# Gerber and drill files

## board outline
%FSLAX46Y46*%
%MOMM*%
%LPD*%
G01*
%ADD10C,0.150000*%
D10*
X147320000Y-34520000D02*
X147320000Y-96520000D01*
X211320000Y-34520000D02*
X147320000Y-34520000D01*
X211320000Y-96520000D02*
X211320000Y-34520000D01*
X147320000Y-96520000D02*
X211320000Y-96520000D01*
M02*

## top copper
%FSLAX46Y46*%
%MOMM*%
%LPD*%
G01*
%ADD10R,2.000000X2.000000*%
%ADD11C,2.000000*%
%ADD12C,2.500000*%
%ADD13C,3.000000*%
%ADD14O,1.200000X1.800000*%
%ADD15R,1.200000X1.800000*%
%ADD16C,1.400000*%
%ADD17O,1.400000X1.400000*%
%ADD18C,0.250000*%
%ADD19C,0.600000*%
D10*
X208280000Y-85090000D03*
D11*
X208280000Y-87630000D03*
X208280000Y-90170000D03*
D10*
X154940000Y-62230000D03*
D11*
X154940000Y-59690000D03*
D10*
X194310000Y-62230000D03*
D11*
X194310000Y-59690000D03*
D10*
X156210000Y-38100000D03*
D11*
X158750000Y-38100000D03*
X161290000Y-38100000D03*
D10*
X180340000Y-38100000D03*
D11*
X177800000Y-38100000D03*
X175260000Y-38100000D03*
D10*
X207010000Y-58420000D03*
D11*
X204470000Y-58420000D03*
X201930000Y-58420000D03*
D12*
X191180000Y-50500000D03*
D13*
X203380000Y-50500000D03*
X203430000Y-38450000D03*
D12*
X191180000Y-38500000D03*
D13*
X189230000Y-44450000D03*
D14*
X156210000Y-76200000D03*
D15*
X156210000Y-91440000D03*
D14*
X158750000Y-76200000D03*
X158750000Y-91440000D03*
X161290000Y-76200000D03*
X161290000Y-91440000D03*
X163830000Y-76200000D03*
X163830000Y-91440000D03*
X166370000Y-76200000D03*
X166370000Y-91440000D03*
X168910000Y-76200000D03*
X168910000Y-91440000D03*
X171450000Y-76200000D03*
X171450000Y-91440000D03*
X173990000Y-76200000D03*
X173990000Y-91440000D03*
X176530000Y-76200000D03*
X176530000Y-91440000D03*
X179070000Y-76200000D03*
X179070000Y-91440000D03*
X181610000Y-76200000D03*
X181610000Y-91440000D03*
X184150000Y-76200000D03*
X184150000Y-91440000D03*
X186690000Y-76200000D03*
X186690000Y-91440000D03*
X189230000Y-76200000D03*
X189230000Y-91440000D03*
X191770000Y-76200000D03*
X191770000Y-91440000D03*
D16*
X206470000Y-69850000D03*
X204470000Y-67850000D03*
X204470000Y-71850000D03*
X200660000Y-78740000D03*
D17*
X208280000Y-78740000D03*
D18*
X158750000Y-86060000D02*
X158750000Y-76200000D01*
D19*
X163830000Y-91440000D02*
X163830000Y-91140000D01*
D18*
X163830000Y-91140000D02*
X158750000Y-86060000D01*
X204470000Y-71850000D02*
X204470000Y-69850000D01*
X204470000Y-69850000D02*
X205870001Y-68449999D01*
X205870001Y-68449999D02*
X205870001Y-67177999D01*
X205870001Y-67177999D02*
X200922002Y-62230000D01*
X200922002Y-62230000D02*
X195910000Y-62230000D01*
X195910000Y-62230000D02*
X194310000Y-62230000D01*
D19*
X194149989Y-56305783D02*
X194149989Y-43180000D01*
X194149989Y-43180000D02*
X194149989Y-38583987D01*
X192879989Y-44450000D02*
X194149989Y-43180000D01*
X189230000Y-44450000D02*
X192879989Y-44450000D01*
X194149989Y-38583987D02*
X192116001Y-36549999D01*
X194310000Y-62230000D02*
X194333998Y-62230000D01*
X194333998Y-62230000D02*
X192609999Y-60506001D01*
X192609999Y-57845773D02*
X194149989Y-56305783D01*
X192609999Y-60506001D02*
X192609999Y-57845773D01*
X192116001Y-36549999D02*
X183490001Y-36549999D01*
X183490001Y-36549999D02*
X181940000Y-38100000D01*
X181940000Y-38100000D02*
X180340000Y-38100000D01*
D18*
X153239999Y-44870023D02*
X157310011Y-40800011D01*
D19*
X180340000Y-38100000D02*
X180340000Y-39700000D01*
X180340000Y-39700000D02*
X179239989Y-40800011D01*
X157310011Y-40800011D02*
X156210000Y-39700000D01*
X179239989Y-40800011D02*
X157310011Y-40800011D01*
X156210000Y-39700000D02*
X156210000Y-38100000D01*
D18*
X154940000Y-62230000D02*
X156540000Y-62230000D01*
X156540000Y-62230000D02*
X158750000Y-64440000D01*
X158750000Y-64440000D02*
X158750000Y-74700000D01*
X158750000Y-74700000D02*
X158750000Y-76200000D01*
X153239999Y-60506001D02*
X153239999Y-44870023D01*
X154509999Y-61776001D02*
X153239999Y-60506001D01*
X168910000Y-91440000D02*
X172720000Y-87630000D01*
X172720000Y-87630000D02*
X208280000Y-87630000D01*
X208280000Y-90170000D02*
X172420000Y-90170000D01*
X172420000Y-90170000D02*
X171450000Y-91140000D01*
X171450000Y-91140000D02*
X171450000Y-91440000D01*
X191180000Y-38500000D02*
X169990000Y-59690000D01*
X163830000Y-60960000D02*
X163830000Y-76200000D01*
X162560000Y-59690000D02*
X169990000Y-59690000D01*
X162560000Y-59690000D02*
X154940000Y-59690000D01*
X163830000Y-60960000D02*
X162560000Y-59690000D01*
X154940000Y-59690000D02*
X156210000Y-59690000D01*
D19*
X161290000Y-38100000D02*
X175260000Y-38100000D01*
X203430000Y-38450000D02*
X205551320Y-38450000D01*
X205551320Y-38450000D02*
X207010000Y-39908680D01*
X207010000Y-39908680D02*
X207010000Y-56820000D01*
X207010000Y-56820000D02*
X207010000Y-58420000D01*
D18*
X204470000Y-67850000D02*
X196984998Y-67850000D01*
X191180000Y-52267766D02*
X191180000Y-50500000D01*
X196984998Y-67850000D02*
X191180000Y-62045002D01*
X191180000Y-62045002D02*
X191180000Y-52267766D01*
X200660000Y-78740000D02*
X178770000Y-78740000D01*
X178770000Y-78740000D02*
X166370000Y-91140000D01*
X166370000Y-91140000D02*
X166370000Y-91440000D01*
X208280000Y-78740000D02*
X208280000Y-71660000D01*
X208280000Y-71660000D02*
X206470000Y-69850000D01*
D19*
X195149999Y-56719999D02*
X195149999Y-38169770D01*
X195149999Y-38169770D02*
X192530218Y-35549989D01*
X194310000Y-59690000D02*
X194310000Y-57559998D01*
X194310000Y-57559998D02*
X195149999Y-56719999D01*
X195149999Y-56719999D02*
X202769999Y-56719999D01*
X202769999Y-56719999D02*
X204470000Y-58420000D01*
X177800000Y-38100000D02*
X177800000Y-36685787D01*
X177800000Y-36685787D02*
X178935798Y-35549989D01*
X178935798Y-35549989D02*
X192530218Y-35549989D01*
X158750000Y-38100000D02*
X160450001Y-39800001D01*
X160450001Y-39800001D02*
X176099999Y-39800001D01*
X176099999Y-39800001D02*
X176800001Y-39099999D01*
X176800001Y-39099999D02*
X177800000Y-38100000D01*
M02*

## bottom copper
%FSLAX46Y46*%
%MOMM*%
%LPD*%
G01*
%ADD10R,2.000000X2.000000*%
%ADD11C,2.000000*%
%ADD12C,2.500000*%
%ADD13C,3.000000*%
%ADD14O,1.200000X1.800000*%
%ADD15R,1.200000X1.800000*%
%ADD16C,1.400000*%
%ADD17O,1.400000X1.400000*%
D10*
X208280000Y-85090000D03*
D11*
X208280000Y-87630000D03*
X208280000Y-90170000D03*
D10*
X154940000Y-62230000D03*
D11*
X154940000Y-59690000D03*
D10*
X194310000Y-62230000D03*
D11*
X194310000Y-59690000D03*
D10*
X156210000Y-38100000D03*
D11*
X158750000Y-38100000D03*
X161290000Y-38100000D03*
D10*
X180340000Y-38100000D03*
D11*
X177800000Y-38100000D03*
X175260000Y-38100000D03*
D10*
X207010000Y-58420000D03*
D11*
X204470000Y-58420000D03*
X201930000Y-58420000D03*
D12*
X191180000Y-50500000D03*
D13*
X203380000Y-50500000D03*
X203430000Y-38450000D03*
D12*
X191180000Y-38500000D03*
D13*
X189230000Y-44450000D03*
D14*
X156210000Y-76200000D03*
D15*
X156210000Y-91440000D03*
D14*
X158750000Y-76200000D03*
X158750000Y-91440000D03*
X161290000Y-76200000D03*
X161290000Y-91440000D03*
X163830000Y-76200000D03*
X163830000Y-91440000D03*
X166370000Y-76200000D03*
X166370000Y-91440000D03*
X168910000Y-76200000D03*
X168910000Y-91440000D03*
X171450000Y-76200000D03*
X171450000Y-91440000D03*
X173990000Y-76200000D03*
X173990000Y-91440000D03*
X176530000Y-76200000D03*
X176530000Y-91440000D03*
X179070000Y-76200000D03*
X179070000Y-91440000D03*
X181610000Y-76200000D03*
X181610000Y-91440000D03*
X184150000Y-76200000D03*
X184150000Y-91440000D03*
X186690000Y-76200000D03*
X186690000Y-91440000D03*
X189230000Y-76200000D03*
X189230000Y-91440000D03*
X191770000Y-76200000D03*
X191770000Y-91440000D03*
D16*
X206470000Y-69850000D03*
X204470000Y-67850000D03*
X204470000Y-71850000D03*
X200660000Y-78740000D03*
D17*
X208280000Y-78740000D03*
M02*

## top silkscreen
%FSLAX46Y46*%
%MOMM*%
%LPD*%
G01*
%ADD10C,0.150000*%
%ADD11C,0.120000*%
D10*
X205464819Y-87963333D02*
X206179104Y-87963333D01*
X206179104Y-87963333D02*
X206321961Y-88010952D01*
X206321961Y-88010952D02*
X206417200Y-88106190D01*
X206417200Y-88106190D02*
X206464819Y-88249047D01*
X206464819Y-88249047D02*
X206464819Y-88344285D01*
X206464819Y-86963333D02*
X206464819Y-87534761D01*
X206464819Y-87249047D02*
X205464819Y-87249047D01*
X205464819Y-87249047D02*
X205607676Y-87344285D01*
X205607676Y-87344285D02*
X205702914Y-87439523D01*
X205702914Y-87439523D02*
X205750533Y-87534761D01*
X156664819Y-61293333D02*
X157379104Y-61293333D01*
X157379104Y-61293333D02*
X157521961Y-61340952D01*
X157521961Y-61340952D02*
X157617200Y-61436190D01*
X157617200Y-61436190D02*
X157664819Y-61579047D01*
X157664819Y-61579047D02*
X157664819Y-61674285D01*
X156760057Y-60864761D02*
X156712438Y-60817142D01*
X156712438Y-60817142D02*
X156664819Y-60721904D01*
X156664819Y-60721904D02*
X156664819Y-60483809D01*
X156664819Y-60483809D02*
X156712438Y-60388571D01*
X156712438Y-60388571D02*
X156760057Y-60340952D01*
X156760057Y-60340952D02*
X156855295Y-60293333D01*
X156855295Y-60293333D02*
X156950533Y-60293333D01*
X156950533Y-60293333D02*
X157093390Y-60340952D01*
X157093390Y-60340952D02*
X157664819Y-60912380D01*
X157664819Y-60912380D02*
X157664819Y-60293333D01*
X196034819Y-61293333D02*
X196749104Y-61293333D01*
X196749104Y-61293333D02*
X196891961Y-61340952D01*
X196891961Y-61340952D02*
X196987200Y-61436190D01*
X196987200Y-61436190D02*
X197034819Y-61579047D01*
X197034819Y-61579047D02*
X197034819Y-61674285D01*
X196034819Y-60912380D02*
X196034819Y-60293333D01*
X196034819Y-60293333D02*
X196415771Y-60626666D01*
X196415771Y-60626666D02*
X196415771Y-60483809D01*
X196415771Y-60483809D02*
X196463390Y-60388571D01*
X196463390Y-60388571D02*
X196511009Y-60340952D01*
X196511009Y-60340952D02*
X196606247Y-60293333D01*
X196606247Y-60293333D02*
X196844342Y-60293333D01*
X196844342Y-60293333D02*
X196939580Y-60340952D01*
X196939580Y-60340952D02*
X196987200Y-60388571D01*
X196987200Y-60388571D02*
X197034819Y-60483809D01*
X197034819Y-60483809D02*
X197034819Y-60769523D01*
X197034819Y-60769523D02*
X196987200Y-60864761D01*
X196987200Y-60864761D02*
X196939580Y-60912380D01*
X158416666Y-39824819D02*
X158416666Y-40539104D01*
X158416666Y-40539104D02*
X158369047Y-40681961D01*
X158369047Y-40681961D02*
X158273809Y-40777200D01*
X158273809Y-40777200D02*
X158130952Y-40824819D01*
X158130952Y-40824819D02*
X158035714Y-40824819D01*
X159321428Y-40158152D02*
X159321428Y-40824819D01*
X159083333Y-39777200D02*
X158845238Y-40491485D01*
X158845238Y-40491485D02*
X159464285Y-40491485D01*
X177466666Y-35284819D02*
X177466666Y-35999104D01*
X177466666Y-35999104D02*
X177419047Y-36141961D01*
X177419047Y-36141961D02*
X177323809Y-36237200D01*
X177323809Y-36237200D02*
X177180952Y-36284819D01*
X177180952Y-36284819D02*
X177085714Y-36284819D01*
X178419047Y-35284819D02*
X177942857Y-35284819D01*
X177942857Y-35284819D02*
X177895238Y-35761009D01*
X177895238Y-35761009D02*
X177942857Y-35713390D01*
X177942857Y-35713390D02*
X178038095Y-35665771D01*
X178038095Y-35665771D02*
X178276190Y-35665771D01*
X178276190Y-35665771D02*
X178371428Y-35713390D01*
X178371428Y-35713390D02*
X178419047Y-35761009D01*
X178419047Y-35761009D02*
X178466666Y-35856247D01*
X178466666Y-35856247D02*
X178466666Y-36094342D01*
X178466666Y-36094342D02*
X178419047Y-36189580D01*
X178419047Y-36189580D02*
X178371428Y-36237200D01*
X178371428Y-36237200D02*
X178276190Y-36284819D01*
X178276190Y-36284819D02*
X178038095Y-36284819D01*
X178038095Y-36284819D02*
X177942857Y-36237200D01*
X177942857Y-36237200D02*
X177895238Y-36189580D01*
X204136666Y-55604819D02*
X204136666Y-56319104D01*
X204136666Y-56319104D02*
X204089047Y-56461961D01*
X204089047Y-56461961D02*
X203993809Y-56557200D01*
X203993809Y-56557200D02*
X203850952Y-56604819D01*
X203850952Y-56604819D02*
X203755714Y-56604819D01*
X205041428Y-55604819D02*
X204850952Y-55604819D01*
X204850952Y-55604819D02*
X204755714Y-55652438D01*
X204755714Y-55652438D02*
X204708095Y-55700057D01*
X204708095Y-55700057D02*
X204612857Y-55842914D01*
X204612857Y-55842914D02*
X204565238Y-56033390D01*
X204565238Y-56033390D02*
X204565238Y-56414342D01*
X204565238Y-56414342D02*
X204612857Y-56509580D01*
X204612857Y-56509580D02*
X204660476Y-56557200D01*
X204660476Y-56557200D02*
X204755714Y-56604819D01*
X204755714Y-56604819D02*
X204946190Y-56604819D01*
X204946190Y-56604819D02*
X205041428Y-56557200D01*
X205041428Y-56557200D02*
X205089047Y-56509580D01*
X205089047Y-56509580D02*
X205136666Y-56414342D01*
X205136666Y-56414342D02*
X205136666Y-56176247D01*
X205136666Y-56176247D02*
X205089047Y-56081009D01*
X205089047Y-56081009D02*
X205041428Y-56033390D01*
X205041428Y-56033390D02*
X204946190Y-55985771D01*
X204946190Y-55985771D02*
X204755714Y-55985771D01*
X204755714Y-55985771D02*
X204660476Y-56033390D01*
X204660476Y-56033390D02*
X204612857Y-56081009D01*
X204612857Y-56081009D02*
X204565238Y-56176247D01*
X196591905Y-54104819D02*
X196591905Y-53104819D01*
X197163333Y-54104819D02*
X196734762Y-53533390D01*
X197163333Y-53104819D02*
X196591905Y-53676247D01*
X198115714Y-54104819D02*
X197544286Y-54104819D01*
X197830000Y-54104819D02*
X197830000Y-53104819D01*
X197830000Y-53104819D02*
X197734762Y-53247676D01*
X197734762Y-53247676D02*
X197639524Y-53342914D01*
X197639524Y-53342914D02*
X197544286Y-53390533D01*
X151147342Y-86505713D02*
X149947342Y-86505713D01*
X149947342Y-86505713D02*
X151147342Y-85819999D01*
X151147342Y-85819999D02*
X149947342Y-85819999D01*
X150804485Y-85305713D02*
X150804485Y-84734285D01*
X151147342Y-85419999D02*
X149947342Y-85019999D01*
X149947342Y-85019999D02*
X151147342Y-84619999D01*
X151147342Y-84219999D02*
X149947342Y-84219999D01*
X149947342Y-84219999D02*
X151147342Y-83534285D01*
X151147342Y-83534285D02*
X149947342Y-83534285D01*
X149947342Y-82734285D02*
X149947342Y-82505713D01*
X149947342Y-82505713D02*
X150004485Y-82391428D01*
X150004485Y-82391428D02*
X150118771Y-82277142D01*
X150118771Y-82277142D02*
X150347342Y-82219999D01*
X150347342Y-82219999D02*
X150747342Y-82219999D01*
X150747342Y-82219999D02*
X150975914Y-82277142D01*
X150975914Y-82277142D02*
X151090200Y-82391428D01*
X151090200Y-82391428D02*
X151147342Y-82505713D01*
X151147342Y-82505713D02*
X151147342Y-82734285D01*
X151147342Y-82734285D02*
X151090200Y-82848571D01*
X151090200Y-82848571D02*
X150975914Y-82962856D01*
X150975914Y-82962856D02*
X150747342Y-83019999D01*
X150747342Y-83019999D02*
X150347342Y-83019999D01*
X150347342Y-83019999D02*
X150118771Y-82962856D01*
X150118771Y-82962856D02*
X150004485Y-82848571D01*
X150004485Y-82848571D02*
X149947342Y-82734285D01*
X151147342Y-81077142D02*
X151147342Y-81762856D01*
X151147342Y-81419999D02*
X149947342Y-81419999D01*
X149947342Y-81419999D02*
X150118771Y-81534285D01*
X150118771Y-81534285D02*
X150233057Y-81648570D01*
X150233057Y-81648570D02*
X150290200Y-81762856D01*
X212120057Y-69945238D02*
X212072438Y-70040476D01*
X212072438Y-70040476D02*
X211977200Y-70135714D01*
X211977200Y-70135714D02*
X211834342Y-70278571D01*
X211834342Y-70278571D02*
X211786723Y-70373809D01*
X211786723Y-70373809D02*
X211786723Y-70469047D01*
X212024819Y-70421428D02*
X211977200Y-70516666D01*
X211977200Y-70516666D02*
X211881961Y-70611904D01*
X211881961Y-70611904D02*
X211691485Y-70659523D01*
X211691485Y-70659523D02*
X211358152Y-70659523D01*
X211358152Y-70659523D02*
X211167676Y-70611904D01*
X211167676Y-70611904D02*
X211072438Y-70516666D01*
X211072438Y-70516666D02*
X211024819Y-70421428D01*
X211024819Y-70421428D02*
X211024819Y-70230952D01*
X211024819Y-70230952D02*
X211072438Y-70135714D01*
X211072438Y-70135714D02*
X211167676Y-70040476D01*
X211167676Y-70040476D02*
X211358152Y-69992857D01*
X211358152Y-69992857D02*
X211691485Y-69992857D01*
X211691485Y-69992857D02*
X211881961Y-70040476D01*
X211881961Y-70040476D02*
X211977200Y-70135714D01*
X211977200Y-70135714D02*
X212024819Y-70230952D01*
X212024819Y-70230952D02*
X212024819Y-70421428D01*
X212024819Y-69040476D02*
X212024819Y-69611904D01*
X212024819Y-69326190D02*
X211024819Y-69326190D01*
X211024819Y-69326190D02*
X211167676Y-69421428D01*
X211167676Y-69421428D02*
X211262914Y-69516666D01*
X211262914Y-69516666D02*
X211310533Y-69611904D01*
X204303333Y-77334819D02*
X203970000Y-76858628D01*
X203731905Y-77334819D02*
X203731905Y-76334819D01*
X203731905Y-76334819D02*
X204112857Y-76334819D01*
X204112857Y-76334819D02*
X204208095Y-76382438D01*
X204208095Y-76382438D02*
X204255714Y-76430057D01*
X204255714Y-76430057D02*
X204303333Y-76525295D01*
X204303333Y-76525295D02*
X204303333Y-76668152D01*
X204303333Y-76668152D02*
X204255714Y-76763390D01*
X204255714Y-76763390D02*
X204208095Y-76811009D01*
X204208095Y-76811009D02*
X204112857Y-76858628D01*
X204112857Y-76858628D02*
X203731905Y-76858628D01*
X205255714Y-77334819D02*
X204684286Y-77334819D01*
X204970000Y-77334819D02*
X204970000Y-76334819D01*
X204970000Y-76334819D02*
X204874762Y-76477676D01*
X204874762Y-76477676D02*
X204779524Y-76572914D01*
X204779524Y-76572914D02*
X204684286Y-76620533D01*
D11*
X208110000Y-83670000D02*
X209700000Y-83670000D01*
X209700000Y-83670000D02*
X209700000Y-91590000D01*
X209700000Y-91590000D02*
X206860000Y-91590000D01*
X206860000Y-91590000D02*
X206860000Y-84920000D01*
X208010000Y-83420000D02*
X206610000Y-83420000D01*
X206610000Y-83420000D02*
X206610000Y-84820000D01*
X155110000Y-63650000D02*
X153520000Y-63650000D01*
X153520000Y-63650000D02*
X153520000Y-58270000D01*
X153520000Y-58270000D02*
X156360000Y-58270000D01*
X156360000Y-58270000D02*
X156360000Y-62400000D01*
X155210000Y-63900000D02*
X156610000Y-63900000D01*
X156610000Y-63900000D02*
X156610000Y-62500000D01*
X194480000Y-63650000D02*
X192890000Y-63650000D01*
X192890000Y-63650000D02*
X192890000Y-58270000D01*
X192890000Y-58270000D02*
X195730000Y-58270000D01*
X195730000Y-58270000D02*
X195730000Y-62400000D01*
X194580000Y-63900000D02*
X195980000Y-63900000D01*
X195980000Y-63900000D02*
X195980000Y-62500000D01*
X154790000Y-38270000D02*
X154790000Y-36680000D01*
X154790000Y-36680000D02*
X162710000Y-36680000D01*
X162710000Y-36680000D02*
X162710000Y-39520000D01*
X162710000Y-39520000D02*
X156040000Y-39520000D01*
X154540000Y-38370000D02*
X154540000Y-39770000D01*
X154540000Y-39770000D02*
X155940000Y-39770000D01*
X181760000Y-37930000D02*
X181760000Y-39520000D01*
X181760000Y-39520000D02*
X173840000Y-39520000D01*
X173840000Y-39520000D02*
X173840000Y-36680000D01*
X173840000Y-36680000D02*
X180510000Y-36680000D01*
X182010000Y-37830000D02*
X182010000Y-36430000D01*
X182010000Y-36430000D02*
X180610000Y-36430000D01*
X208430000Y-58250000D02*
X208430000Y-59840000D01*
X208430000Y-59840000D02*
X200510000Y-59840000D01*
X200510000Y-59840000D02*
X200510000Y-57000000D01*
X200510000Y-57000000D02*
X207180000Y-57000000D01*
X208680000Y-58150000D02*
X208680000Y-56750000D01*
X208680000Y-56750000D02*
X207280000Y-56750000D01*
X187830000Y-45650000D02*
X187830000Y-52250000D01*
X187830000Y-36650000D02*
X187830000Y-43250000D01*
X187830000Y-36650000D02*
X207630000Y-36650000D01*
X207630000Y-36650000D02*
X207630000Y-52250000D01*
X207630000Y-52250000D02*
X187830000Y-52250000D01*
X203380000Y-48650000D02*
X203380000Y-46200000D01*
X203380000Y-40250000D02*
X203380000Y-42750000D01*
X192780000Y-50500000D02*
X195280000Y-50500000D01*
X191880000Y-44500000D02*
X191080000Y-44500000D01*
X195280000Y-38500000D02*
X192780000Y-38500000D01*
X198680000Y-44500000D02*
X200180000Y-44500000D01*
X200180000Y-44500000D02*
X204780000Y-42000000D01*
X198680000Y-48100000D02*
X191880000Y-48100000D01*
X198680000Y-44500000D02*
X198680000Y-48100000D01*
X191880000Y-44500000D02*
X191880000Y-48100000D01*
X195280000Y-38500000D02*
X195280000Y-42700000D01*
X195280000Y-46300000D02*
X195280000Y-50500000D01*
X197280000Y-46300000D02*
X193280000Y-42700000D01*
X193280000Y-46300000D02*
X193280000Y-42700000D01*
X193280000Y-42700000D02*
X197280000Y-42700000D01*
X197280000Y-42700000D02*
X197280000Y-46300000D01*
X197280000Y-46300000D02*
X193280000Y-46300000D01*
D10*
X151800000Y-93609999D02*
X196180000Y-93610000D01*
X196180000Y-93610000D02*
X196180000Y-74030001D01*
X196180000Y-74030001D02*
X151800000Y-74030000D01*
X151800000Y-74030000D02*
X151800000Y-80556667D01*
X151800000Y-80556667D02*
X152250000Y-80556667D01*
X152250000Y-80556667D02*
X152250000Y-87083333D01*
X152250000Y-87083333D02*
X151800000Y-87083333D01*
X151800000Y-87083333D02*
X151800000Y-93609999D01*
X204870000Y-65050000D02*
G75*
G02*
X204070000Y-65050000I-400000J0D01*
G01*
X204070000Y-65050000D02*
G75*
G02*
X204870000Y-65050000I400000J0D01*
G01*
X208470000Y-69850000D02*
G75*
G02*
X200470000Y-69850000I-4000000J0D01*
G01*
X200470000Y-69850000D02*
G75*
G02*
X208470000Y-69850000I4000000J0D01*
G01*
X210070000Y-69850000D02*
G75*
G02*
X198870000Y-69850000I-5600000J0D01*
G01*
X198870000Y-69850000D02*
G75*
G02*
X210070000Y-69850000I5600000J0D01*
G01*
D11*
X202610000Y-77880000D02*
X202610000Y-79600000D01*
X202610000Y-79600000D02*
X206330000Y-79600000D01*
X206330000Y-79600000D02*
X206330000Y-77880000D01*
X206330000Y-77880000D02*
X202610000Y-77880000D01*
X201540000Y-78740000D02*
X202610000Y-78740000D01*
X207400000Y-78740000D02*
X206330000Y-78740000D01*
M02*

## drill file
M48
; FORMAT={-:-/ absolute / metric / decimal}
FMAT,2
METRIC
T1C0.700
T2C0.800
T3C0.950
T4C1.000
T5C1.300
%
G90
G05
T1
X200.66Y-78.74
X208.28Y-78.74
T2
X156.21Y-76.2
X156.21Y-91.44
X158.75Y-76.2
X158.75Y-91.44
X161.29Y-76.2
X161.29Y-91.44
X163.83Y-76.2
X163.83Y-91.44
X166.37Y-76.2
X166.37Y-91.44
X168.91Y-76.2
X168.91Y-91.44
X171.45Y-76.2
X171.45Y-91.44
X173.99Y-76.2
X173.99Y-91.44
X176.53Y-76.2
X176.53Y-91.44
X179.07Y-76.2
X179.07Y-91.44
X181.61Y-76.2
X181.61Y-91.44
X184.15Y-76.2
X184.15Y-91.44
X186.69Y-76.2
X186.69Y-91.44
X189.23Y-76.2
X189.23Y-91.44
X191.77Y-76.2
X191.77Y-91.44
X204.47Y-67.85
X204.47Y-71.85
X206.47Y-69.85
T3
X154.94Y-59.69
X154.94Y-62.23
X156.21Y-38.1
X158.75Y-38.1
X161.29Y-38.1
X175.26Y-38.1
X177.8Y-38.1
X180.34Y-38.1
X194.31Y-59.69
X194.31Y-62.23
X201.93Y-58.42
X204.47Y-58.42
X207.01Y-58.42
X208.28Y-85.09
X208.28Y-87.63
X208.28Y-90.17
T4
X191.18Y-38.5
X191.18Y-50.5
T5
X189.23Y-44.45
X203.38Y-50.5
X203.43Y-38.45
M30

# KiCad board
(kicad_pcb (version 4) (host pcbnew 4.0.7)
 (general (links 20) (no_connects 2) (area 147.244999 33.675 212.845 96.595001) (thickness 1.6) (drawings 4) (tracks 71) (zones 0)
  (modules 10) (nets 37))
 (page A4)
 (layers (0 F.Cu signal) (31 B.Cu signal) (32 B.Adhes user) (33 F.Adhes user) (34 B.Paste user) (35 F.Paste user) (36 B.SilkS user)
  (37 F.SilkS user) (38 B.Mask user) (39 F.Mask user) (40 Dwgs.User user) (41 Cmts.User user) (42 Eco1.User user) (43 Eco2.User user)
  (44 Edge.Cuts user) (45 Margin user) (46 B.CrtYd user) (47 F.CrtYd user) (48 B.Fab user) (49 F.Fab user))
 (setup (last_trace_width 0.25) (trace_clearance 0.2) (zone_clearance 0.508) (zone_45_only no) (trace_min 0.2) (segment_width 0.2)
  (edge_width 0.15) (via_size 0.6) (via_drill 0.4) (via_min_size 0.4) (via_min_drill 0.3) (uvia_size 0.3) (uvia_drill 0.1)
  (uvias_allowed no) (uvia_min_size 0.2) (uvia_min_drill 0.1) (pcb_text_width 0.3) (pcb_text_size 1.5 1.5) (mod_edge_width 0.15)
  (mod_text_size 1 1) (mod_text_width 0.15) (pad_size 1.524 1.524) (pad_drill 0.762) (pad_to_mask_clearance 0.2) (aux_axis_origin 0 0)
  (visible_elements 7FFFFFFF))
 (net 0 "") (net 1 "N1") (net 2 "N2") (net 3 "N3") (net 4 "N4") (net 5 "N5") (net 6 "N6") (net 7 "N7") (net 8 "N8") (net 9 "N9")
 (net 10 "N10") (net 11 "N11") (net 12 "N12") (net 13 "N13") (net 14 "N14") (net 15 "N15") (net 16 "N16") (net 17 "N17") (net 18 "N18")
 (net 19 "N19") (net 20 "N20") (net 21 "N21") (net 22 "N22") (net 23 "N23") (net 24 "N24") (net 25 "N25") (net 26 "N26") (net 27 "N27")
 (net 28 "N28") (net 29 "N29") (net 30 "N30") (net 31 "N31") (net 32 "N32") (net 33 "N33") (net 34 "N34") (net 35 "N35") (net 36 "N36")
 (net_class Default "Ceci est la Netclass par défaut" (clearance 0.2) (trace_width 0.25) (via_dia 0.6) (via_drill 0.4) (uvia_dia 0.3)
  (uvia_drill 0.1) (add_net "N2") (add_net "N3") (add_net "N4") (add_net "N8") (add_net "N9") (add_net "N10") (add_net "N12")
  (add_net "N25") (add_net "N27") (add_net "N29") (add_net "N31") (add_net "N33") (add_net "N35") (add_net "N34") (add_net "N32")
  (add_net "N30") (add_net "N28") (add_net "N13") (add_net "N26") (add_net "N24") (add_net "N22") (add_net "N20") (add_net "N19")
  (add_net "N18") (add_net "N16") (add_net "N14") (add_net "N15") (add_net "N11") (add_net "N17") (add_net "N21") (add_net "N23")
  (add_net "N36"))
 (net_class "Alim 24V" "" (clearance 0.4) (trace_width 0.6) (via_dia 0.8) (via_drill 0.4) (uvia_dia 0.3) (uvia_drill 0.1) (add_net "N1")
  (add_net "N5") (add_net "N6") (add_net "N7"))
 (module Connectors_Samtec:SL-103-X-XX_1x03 (layer F.Cu) (at 208.28 85.09)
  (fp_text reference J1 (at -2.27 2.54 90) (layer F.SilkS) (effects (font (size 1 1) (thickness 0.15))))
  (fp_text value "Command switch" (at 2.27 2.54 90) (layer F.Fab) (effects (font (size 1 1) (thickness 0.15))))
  (fp_line (start -0.17 -1.42) (end 1.42 -1.42) (layer F.SilkS) (width 0.12))
  (fp_line (start 1.42 -1.42) (end 1.42 6.5) (layer F.SilkS) (width 0.12))
  (fp_line (start 1.42 6.5) (end -1.42 6.5) (layer F.SilkS) (width 0.12))
  (fp_line (start -1.42 6.5) (end -1.42 -0.17) (layer F.SilkS) (width 0.12))
  (fp_line (start -0.27 -1.67) (end -1.67 -1.67) (layer F.SilkS) (width 0.12))
  (fp_line (start -1.67 -1.67) (end -1.67 -0.27) (layer F.SilkS) (width 0.12))
  (pad 1 thru_hole rect (at 0 0) (size 2 2) (drill 0.95) (layers *.Cu *.Mask) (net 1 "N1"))
  (pad 2 thru_hole circle (at 0 2.54) (size 2 2) (drill 0.95) (layers *.Cu *.Mask) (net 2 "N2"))
  (pad 3 thru_hole circle (at 0 5.08) (size 2 2) (drill 0.95) (layers *.Cu *.Mask) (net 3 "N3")))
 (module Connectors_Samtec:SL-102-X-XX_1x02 (layer F.Cu) (at 154.94 62.23 180)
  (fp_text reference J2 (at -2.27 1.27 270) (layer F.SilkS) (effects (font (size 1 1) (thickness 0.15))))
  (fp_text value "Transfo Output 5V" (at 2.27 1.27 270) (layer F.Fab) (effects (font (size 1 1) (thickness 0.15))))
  (fp_line (start -0.17 -1.42) (end 1.42 -1.42) (layer F.SilkS) (width 0.12))
  (fp_line (start 1.42 -1.42) (end 1.42 3.96) (layer F.SilkS) (width 0.12))
  (fp_line (start 1.42 3.96) (end -1.42 3.96) (layer F.SilkS) (width 0.12))
  (fp_line (start -1.42 3.96) (end -1.42 -0.17) (layer F.SilkS) (width 0.12))
  (fp_line (start -0.27 -1.67) (end -1.67 -1.67) (layer F.SilkS) (width 0.12))
  (fp_line (start -1.67 -1.67) (end -1.67 -0.27) (layer F.SilkS) (width 0.12))
  (pad 1 thru_hole rect (at 0 0 180) (size 2 2) (drill 0.95) (layers *.Cu *.Mask) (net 1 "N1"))
  (pad 2 thru_hole circle (at 0 2.54 180) (size 2 2) (drill 0.95) (layers *.Cu *.Mask) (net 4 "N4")))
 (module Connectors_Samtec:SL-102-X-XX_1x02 (layer F.Cu) (at 194.31 62.23 180)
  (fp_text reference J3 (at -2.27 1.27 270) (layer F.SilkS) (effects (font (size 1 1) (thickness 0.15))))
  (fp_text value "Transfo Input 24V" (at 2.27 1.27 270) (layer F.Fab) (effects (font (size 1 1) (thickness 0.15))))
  (fp_line (start -0.17 -1.42) (end 1.42 -1.42) (layer F.SilkS) (width 0.12))
  (fp_line (start 1.42 -1.42) (end 1.42 3.96) (layer F.SilkS) (width 0.12))
  (fp_line (start 1.42 3.96) (end -1.42 3.96) (layer F.SilkS) (width 0.12))
  (fp_line (start -1.42 3.96) (end -1.42 -0.17) (layer F.SilkS) (width 0.12))
  (fp_line (start -0.27 -1.67) (end -1.67 -1.67) (layer F.SilkS) (width 0.12))
  (fp_line (start -1.67 -1.67) (end -1.67 -0.27) (layer F.SilkS) (width 0.12))
  (pad 1 thru_hole rect (at 0 0 180) (size 2 2) (drill 0.95) (layers *.Cu *.Mask) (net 1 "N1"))
  (pad 2 thru_hole circle (at 0 2.54 180) (size 2 2) (drill 0.95) (layers *.Cu *.Mask) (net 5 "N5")))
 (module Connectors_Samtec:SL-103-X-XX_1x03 (layer F.Cu) (at 156.21 38.1 90)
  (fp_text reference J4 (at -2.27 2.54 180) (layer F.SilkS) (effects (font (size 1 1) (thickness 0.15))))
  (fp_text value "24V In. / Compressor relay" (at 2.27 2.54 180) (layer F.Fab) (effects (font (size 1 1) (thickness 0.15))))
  (fp_line (start -0.17 -1.42) (end 1.42 -1.42) (layer F.SilkS) (width 0.12))
  (fp_line (start 1.42 -1.42) (end 1.42 6.5) (layer F.SilkS) (width 0.12))
  (fp_line (start 1.42 6.5) (end -1.42 6.5) (layer F.SilkS) (width 0.12))
  (fp_line (start -1.42 6.5) (end -1.42 -0.17) (layer F.SilkS) (width 0.12))
  (fp_line (start -0.27 -1.67) (end -1.67 -1.67) (layer F.SilkS) (width 0.12))
  (fp_line (start -1.67 -1.67) (end -1.67 -0.27) (layer F.SilkS) (width 0.12))
  (pad 1 thru_hole rect (at 0 0 90) (size 2 2) (drill 0.95) (layers *.Cu *.Mask) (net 1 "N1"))
  (pad 2 thru_hole circle (at 0 2.54 90) (size 2 2) (drill 0.95) (layers *.Cu *.Mask) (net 5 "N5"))
  (pad 3 thru_hole circle (at 0 5.08 90) (size 2 2) (drill 0.95) (layers *.Cu *.Mask) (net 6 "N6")))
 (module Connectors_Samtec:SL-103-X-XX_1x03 (layer F.Cu) (at 180.34 38.1 270)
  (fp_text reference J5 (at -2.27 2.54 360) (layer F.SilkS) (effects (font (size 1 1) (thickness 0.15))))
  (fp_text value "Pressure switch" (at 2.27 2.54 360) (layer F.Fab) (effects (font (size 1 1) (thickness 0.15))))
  (fp_line (start -0.17 -1.42) (end 1.42 -1.42) (layer F.SilkS) (width 0.12))
  (fp_line (start 1.42 -1.42) (end 1.42 6.5) (layer F.SilkS) (width 0.12))
  (fp_line (start 1.42 6.5) (end -1.42 6.5) (layer F.SilkS) (width 0.12))
  (fp_line (start -1.42 6.5) (end -1.42 -0.17) (layer F.SilkS) (width 0.12))
  (fp_line (start -0.27 -1.67) (end -1.67 -1.67) (layer F.SilkS) (width 0.12))
  (fp_line (start -1.67 -1.67) (end -1.67 -0.27) (layer F.SilkS) (width 0.12))
  (pad 1 thru_hole rect (at 0 0 270) (size 2 2) (drill 0.95) (layers *.Cu *.Mask) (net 1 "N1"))
  (pad 2 thru_hole circle (at 0 2.54 270) (size 2 2) (drill 0.95) (layers *.Cu *.Mask) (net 5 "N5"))
  (pad 3 thru_hole circle (at 0 5.08 270) (size 2 2) (drill 0.95) (layers *.Cu *.Mask) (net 6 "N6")))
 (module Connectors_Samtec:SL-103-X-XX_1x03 (layer F.Cu) (at 207.01 58.42 270)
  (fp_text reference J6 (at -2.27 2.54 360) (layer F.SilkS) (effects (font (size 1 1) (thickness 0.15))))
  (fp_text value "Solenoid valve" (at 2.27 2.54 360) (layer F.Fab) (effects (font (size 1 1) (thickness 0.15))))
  (fp_line (start -0.17 -1.42) (end 1.42 -1.42) (layer F.SilkS) (width 0.12))
  (fp_line (start 1.42 -1.42) (end 1.42 6.5) (layer F.SilkS) (width 0.12))
  (fp_line (start 1.42 6.5) (end -1.42 6.5) (layer F.SilkS) (width 0.12))
  (fp_line (start -1.42 6.5) (end -1.42 -0.17) (layer F.SilkS) (width 0.12))
  (fp_line (start -0.27 -1.67) (end -1.67 -1.67) (layer F.SilkS) (width 0.12))
  (fp_line (start -1.67 -1.67) (end -1.67 -0.27) (layer F.SilkS) (width 0.12))
  (pad 1 thru_hole rect (at 0 0 270) (size 2 2) (drill 0.95) (layers *.Cu *.Mask) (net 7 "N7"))
  (pad 2 thru_hole circle (at 0 2.54 270) (size 2 2) (drill 0.95) (layers *.Cu *.Mask) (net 5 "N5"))
  (pad 3 thru_hole circle (at 0 5.08 270) (size 2 2) (drill 0.95) (layers *.Cu *.Mask) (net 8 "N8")))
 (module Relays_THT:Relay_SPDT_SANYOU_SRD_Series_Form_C (layer F.Cu) (at 189.23 44.45)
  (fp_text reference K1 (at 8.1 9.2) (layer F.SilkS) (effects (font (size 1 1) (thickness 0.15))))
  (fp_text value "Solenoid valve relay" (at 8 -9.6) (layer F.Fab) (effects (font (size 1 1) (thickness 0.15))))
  (fp_line (start -1.4 1.2) (end -1.4 7.8) (layer F.SilkS) (width 0.12))
  (fp_line (start -1.4 -7.8) (end -1.4 -1.2) (layer F.SilkS) (width 0.12))
  (fp_line (start -1.4 -7.8) (end 18.4 -7.8) (layer F.SilkS) (width 0.12))
  (fp_line (start 18.4 -7.8) (end 18.4 7.8) (layer F.SilkS) (width 0.12))
  (fp_line (start 18.4 7.8) (end -1.4 7.8) (layer F.SilkS) (width 0.12))
  (fp_line (start 14.15 4.2) (end 14.15 1.75) (layer F.SilkS) (width 0.12))
  (fp_line (start 14.15 -4.2) (end 14.15 -1.7) (layer F.SilkS) (width 0.12))
  (fp_line (start 3.55 6.05) (end 6.05 6.05) (layer F.SilkS) (width 0.12))
  (fp_line (start 2.65 0.05) (end 1.85 0.05) (layer F.SilkS) (width 0.12))
  (fp_line (start 6.05 -5.95) (end 3.55 -5.95) (layer F.SilkS) (width 0.12))
  (fp_line (start 9.45 0.05) (end 10.95 0.05) (layer F.SilkS) (width 0.12))
  (fp_line (start 10.95 0.05) (end 15.55 -2.45) (layer F.SilkS) (width 0.12))
  (fp_line (start 9.45 3.65) (end 2.65 3.65) (layer F.SilkS) (width 0.12))
  (fp_line (start 9.45 0.05) (end 9.45 3.65) (layer F.SilkS) (width 0.12))
  (fp_line (start 2.65 0.05) (end 2.65 3.65) (layer F.SilkS) (width 0.12))
  (fp_line (start 6.05 -5.95) (end 6.05 -1.75) (layer F.SilkS) (width 0.12))
  (fp_line (start 6.05 1.85) (end 6.05 6.05) (layer F.SilkS) (width 0.12))
  (fp_line (start 8.05 1.85) (end 4.05 -1.75) (layer F.SilkS) (width 0.12))
  (fp_line (start 4.05 1.85) (end 4.05 -1.75) (layer F.SilkS) (width 0.12))
  (fp_line (start 4.05 -1.75) (end 8.05 -1.75) (layer F.SilkS) (width 0.12))
  (fp_line (start 8.05 -1.75) (end 8.05 1.85) (layer F.SilkS) (width 0.12))
  (fp_line (start 8.05 1.85) (end 4.05 1.85) (layer F.SilkS) (width 0.12))
  (pad 2 thru_hole circle (at 1.95 6.05 90) (size 2.5 2.5) (drill 1) (layers *.Cu *.Mask) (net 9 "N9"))
  (pad 3 thru_hole circle (at 14.15 6.05 90) (size 3 3) (drill 1.3) (layers *.Cu *.Mask) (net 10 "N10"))
  (pad 4 thru_hole circle (at 14.2 -6 90) (size 3 3) (drill 1.3) (layers *.Cu *.Mask) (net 7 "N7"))
  (pad 5 thru_hole circle (at 1.95 -5.95 90) (size 2.5 2.5) (drill 1) (layers *.Cu *.Mask) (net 4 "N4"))
  (pad 1 thru_hole circle (at 0 0 90) (size 3 3) (drill 1.3) (layers *.Cu *.Mask) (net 1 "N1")))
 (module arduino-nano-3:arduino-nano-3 (layer F.Cu) (at 173.99 83.82)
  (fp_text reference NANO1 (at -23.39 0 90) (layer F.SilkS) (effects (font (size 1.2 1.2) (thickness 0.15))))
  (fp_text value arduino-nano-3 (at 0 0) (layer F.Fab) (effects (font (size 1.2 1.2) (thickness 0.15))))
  (fp_line (start -22.19 9.789999) (end 22.19 9.79) (layer F.SilkS) (width 0.15))
  (fp_line (start 22.19 9.79) (end 22.19 -9.789999) (layer F.SilkS) (width 0.15))
  (fp_line (start 22.19 -9.789999) (end -22.19 -9.79) (layer F.SilkS) (width 0.15))
  (fp_line (start -22.19 -9.79) (end -22.19 -3.263333) (layer F.SilkS) (width 0.15))
  (fp_line (start -22.19 -3.263333) (end -21.74 -3.263333) (layer F.SilkS) (width 0.15))
  (fp_line (start -21.74 -3.263333) (end -21.74 3.263333) (layer F.SilkS) (width 0.15))
  (fp_line (start -21.74 3.263333) (end -22.19 3.263333) (layer F.SilkS) (width 0.15))
  (fp_line (start -22.19 3.263333) (end -22.19 9.789999) (layer F.SilkS) (width 0.15))
  (pad 30 thru_hole oval (at -17.78 -7.62) (size 1.2 1.8) (drill 0.8) (layers *.Cu *.Mask) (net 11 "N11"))
  (pad 1 thru_hole rect (at -17.78 7.62) (size 1.2 1.8) (drill 0.8) (layers *.Cu *.Mask) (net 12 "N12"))
  (pad 29 thru_hole oval (at -15.24 -7.62) (size 1.2 1.8) (drill 0.8) (layers *.Cu *.Mask) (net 1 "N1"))
  (pad 2 thru_hole oval (at -15.24 7.62) (size 1.2 1.8) (drill 0.8) (layers *.Cu *.Mask) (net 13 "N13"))
  (pad 28 thru_hole oval (at -12.7 -7.62) (size 1.2 1.8) (drill 0.8) (layers *.Cu *.Mask) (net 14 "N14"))
  (pad 3 thru_hole oval (at -12.7 7.62) (size 1.2 1.8) (drill 0.8) (layers *.Cu *.Mask) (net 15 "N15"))
  (pad 27 thru_hole oval (at -10.16 -7.62) (size 1.2 1.8) (drill 0.8) (layers *.Cu *.Mask) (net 4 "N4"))
  (pad 4 thru_hole oval (at -10.16 7.62) (size 1.2 1.8) (drill 0.8) (layers *.Cu *.Mask) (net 1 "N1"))
  (pad 26 thru_hole oval (at -7.62 -7.62) (size 1.2 1.8) (drill 0.8) (layers *.Cu *.Mask) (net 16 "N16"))
  (pad 5 thru_hole oval (at -7.62 7.62) (size 1.2 1.8) (drill 0.8) (layers *.Cu *.Mask) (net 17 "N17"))
  (pad 25 thru_hole oval (at -5.08 -7.62) (size 1.2 1.8) (drill 0.8) (layers *.Cu *.Mask) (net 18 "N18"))
  (pad 6 thru_hole oval (at -5.08 7.62) (size 1.2 1.8) (drill 0.8) (layers *.Cu *.Mask) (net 2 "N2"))
  (pad 24 thru_hole oval (at -2.54 -7.62) (size 1.2 1.8) (drill 0.8) (layers *.Cu *.Mask) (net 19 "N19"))
  (pad 7 thru_hole oval (at -2.54 7.62) (size 1.2 1.8) (drill 0.8) (layers *.Cu *.Mask) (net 3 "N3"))
  (pad 23 thru_hole oval (at 0 -7.62) (size 1.2 1.8) (drill 0.8) (layers *.Cu *.Mask) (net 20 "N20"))
  (pad 8 thru_hole oval (at 0 7.62) (size 1.2 1.8) (drill 0.8) (layers *.Cu *.Mask) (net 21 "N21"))
  (pad 22 thru_hole oval (at 2.54 -7.62) (size 1.2 1.8) (drill 0.8) (layers *.Cu *.Mask) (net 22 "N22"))
  (pad 9 thru_hole oval (at 2.54 7.62) (size 1.2 1.8) (drill 0.8) (layers *.Cu *.Mask) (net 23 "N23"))
  (pad 21 thru_hole oval (at 5.08 -7.62) (size 1.2 1.8) (drill 0.8) (layers *.Cu *.Mask) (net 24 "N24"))
  (pad 10 thru_hole oval (at 5.08 7.62) (size 1.2 1.8) (drill 0.8) (layers *.Cu *.Mask) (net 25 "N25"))
  (pad 20 thru_hole oval (at 7.62 -7.62) (size 1.2 1.8) (drill 0.8) (layers *.Cu *.Mask) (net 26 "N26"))
  (pad 11 thru_hole oval (at 7.62 7.62) (size 1.2 1.8) (drill 0.8) (layers *.Cu *.Mask) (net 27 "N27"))
  (pad 19 thru_hole oval (at 10.16 -7.62) (size 1.2 1.8) (drill 0.8) (layers *.Cu *.Mask) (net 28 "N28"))
  (pad 12 thru_hole oval (at 10.16 7.62) (size 1.2 1.8) (drill 0.8) (layers *.Cu *.Mask) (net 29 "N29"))
  (pad 18 thru_hole oval (at 12.7 -7.62) (size 1.2 1.8) (drill 0.8) (layers *.Cu *.Mask) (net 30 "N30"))
  (pad 13 thru_hole oval (at 12.7 7.62) (size 1.2 1.8) (drill 0.8) (layers *.Cu *.Mask) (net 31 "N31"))
  (pad 17 thru_hole oval (at 15.24 -7.62) (size 1.2 1.8) (drill 0.8) (layers *.Cu *.Mask) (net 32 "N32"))
  (pad 14 thru_hole oval (at 15.24 7.62) (size 1.2 1.8) (drill 0.8) (layers *.Cu *.Mask) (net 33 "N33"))
  (pad 16 thru_hole oval (at 17.78 -7.62) (size 1.2 1.8) (drill 0.8) (layers *.Cu *.Mask) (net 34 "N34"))
  (pad 15 thru_hole oval (at 17.78 7.62) (size 1.2 1.8) (drill 0.8) (layers *.Cu *.Mask) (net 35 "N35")))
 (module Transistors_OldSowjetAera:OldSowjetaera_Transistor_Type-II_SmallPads (layer F.Cu) (at 204.47 69.85 270)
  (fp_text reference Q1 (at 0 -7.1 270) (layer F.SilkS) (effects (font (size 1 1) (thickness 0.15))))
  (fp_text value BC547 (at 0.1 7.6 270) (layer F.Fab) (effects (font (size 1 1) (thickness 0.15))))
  (fp_circle (center -4.8 0) (end -4.8 0.4) (layer F.SilkS) (width 0.15))
  (fp_circle (center 0 0) (end 4 0) (layer F.SilkS) (width 0.15))
  (fp_circle (center 0 0) (end 5.6 0) (layer F.SilkS) (width 0.15))
  (pad 2 thru_hole circle (at 0 -2 270) (size 1.4 1.4) (drill 0.8) (layers *.Cu *.Mask) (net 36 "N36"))
  (pad 1 thru_hole circle (at -2 0 270) (size 1.4 1.4) (drill 0.8) (layers *.Cu *.Mask) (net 9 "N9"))
  (pad 3 thru_hole circle (at 2 0 270) (size 1.4 1.4) (drill 0.8) (layers *.Cu *.Mask) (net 1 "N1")))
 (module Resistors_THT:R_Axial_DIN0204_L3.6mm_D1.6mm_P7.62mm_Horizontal (layer F.Cu) (at 200.66 78.74)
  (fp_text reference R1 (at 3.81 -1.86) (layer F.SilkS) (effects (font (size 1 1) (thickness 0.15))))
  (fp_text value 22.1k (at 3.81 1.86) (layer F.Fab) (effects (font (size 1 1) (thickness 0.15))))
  (fp_line (start 1.95 -0.86) (end 1.95 0.86) (layer F.SilkS) (width 0.12))
  (fp_line (start 1.95 0.86) (end 5.67 0.86) (layer F.SilkS) (width 0.12))
  (fp_line (start 5.67 0.86) (end 5.67 -0.86) (layer F.SilkS) (width 0.12))
  (fp_line (start 5.67 -0.86) (end 1.95 -0.86) (layer F.SilkS) (width 0.12))
  (fp_line (start 0.88 0) (end 1.95 0) (layer F.SilkS) (width 0.12))
  (fp_line (start 6.74 0) (end 5.67 0) (layer F.SilkS) (width 0.12))
  (pad 1 thru_hole circle (at 0 0) (size 1.4 1.4) (drill 0.7) (layers *.Cu *.Mask) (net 17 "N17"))
  (pad 2 thru_hole oval (at 7.62 0) (size 1.4 1.4) (drill 0.7) (layers *.Cu *.Mask) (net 36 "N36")))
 (gr_line (start 147.32 34.52) (end 147.32 96.52) (angle 90) (layer Edge.Cuts) (width 0.15))
 (gr_line (start 211.32 34.52) (end 147.32 34.52) (angle 90) (layer Edge.Cuts) (width 0.15))
 (gr_line (start 211.32 96.52) (end 211.32 34.52) (angle 90) (layer Edge.Cuts) (width 0.15))
 (gr_line (start 147.32 96.52) (end 211.32 96.52) (angle 90) (layer Edge.Cuts) (width 0.15))
 (segment (start 158.75 86.06) (end 158.75 76.2) (width 0.25) (layer F.Cu) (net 1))
 (segment (start 163.83 91.44) (end 163.83 91.14) (width 0.6) (layer F.Cu) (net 1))
 (segment (start 163.83 91.14) (end 158.75 86.06) (width 0.25) (layer F.Cu) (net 1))
 (segment (start 204.47 71.85) (end 204.47 69.85) (width 0.25) (layer F.Cu) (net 1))
 (segment (start 204.47 69.85) (end 205.870001 68.449999) (width 0.25) (layer F.Cu) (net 1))
 (segment (start 205.870001 68.449999) (end 205.870001 67.177999) (width 0.25) (layer F.Cu) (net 1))
 (segment (start 205.870001 67.177999) (end 200.922002 62.23) (width 0.25) (layer F.Cu) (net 1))
 (segment (start 200.922002 62.23) (end 195.91 62.23) (width 0.25) (layer F.Cu) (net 1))
 (segment (start 195.91 62.23) (end 194.31 62.23) (width 0.25) (layer F.Cu) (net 1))
 (segment (start 194.149989 56.305783) (end 194.149989 43.18) (width 0.6) (layer F.Cu) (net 1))
 (segment (start 194.149989 43.18) (end 194.149989 38.583987) (width 0.6) (layer F.Cu) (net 1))
 (segment (start 192.879989 44.45) (end 194.149989 43.18) (width 0.6) (layer F.Cu) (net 1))
 (segment (start 189.23 44.45) (end 192.879989 44.45) (width 0.6) (layer F.Cu) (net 1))
 (segment (start 194.149989 38.583987) (end 192.116001 36.549999) (width 0.6) (layer F.Cu) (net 1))
 (segment (start 194.31 62.23) (end 194.333998 62.23) (width 0.6) (layer F.Cu) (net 1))
 (segment (start 194.333998 62.23) (end 192.609999 60.506001) (width 0.6) (layer F.Cu) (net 1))
 (segment (start 192.609999 57.845773) (end 194.149989 56.305783) (width 0.6) (layer F.Cu) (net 1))
 (segment (start 192.609999 60.506001) (end 192.609999 57.845773) (width 0.6) (layer F.Cu) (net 1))
 (segment (start 192.116001 36.549999) (end 183.490001 36.549999) (width 0.6) (layer F.Cu) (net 1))
 (segment (start 183.490001 36.549999) (end 181.94 38.1) (width 0.6) (layer F.Cu) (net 1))
 (segment (start 181.94 38.1) (end 180.34 38.1) (width 0.6) (layer F.Cu) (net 1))
 (segment (start 153.239999 44.870023) (end 157.310011 40.800011) (width 0.25) (layer F.Cu) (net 1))
 (segment (start 180.34 38.1) (end 180.34 39.7) (width 0.6) (layer F.Cu) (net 1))
 (segment (start 180.34 39.7) (end 179.239989 40.800011) (width 0.6) (layer F.Cu) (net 1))
 (segment (start 157.310011 40.800011) (end 156.21 39.7) (width 0.6) (layer F.Cu) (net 1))
 (segment (start 179.239989 40.800011) (end 157.310011 40.800011) (width 0.6) (layer F.Cu) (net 1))
 (segment (start 156.21 39.7) (end 156.21 38.1) (width 0.6) (layer F.Cu) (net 1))
 (segment (start 154.94 62.23) (end 156.54 62.23) (width 0.25) (layer F.Cu) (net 1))
 (segment (start 156.54 62.23) (end 158.75 64.44) (width 0.25) (layer F.Cu) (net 1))
 (segment (start 158.75 64.44) (end 158.75 74.7) (width 0.25) (layer F.Cu) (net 1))
 (segment (start 158.75 74.7) (end 158.75 76.2) (width 0.25) (layer F.Cu) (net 1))
 (segment (start 153.239999 60.506001) (end 153.239999 44.870023) (width 0.25) (layer F.Cu) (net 1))
 (segment (start 154.509999 61.776001) (end 153.239999 60.506001) (width 0.25) (layer F.Cu) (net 1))
 (segment (start 168.91 91.44) (end 172.72 87.63) (width 0.25) (layer F.Cu) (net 2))
 (segment (start 172.72 87.63) (end 208.28 87.63) (width 0.25) (layer F.Cu) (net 2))
 (segment (start 208.28 90.17) (end 172.42 90.17) (width 0.25) (layer F.Cu) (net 3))
 (segment (start 172.42 90.17) (end 171.45 91.14) (width 0.25) (layer F.Cu) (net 3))
 (segment (start 171.45 91.14) (end 171.45 91.44) (width 0.25) (layer F.Cu) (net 3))
 (segment (start 191.18 38.5) (end 169.99 59.69) (width 0.25) (layer F.Cu) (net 4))
 (segment (start 163.83 60.96) (end 163.83 76.2) (width 0.25) (layer F.Cu) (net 4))
 (segment (start 162.56 59.69) (end 169.99 59.69) (width 0.25) (layer F.Cu) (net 4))
 (segment (start 162.56 59.69) (end 154.94 59.69) (width 0.25) (layer F.Cu) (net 4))
 (segment (start 163.83 60.96) (end 162.56 59.69) (width 0.25) (layer F.Cu) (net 4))
 (segment (start 154.94 59.69) (end 156.21 59.69) (width 0.25) (layer F.Cu) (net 4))
 (segment (start 161.29 38.1) (end 175.26 38.1) (width 0.6) (layer F.Cu) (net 6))
 (segment (start 203.43 38.45) (end 205.55132 38.45) (width 0.6) (layer F.Cu) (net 7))
 (segment (start 205.55132 38.45) (end 207.01 39.90868) (width 0.6) (layer F.Cu) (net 7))
 (segment (start 207.01 39.90868) (end 207.01 56.82) (width 0.6) (layer F.Cu) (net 7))
 (segment (start 207.01 56.82) (end 207.01 58.42) (width 0.6) (layer F.Cu) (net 7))
 (segment (start 204.47 67.85) (end 196.984998 67.85) (width 0.25) (layer F.Cu) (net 9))
 (segment (start 191.18 52.267766) (end 191.18 50.5) (width 0.25) (layer F.Cu) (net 9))
 (segment (start 196.984998 67.85) (end 191.18 62.045002) (width 0.25) (layer F.Cu) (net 9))
 (segment (start 191.18 62.045002) (end 191.18 52.267766) (width 0.25) (layer F.Cu) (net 9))
 (segment (start 200.66 78.74) (end 178.77 78.74) (width 0.25) (layer F.Cu) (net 17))
 (segment (start 178.77 78.74) (end 166.37 91.14) (width 0.25) (layer F.Cu) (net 17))
 (segment (start 166.37 91.14) (end 166.37 91.44) (width 0.25) (layer F.Cu) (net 17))
 (segment (start 208.28 78.74) (end 208.28 71.66) (width 0.25) (layer F.Cu) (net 36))
 (segment (start 208.28 71.66) (end 206.47 69.85) (width 0.25) (layer F.Cu) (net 36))
 (segment (start 195.149999 56.719999) (end 195.149999 38.16977) (width 0.6) (layer F.Cu) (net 5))
 (segment (start 195.149999 38.16977) (end 192.530218 35.549989) (width 0.6) (layer F.Cu) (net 5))
 (segment (start 194.31 59.69) (end 194.31 57.559998) (width 0.6) (layer F.Cu) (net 5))
 (segment (start 194.31 57.559998) (end 195.149999 56.719999) (width 0.6) (layer F.Cu) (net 5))
 (segment (start 195.149999 56.719999) (end 202.769999 56.719999) (width 0.6) (layer F.Cu) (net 5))
 (segment (start 202.769999 56.719999) (end 204.47 58.42) (width 0.6) (layer F.Cu) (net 5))
 (segment (start 177.8 38.1) (end 177.8 36.685787) (width 0.6) (layer F.Cu) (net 5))
 (segment (start 177.8 36.685787) (end 178.935798 35.549989) (width 0.6) (layer F.Cu) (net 5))
 (segment (start 178.935798 35.549989) (end 192.530218 35.549989) (width 0.6) (layer F.Cu) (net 5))
 (segment (start 158.75 38.1) (end 160.450001 39.800001) (width 0.6) (layer F.Cu) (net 5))
 (segment (start 160.450001 39.800001) (end 176.099999 39.800001) (width 0.6) (layer F.Cu) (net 5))
 (segment (start 176.099999 39.800001) (end 176.800001 39.099999) (width 0.6) (layer F.Cu) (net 5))
 (segment (start 176.800001 39.099999) (end 177.8 38.1) (width 0.6) (layer F.Cu) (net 5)))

